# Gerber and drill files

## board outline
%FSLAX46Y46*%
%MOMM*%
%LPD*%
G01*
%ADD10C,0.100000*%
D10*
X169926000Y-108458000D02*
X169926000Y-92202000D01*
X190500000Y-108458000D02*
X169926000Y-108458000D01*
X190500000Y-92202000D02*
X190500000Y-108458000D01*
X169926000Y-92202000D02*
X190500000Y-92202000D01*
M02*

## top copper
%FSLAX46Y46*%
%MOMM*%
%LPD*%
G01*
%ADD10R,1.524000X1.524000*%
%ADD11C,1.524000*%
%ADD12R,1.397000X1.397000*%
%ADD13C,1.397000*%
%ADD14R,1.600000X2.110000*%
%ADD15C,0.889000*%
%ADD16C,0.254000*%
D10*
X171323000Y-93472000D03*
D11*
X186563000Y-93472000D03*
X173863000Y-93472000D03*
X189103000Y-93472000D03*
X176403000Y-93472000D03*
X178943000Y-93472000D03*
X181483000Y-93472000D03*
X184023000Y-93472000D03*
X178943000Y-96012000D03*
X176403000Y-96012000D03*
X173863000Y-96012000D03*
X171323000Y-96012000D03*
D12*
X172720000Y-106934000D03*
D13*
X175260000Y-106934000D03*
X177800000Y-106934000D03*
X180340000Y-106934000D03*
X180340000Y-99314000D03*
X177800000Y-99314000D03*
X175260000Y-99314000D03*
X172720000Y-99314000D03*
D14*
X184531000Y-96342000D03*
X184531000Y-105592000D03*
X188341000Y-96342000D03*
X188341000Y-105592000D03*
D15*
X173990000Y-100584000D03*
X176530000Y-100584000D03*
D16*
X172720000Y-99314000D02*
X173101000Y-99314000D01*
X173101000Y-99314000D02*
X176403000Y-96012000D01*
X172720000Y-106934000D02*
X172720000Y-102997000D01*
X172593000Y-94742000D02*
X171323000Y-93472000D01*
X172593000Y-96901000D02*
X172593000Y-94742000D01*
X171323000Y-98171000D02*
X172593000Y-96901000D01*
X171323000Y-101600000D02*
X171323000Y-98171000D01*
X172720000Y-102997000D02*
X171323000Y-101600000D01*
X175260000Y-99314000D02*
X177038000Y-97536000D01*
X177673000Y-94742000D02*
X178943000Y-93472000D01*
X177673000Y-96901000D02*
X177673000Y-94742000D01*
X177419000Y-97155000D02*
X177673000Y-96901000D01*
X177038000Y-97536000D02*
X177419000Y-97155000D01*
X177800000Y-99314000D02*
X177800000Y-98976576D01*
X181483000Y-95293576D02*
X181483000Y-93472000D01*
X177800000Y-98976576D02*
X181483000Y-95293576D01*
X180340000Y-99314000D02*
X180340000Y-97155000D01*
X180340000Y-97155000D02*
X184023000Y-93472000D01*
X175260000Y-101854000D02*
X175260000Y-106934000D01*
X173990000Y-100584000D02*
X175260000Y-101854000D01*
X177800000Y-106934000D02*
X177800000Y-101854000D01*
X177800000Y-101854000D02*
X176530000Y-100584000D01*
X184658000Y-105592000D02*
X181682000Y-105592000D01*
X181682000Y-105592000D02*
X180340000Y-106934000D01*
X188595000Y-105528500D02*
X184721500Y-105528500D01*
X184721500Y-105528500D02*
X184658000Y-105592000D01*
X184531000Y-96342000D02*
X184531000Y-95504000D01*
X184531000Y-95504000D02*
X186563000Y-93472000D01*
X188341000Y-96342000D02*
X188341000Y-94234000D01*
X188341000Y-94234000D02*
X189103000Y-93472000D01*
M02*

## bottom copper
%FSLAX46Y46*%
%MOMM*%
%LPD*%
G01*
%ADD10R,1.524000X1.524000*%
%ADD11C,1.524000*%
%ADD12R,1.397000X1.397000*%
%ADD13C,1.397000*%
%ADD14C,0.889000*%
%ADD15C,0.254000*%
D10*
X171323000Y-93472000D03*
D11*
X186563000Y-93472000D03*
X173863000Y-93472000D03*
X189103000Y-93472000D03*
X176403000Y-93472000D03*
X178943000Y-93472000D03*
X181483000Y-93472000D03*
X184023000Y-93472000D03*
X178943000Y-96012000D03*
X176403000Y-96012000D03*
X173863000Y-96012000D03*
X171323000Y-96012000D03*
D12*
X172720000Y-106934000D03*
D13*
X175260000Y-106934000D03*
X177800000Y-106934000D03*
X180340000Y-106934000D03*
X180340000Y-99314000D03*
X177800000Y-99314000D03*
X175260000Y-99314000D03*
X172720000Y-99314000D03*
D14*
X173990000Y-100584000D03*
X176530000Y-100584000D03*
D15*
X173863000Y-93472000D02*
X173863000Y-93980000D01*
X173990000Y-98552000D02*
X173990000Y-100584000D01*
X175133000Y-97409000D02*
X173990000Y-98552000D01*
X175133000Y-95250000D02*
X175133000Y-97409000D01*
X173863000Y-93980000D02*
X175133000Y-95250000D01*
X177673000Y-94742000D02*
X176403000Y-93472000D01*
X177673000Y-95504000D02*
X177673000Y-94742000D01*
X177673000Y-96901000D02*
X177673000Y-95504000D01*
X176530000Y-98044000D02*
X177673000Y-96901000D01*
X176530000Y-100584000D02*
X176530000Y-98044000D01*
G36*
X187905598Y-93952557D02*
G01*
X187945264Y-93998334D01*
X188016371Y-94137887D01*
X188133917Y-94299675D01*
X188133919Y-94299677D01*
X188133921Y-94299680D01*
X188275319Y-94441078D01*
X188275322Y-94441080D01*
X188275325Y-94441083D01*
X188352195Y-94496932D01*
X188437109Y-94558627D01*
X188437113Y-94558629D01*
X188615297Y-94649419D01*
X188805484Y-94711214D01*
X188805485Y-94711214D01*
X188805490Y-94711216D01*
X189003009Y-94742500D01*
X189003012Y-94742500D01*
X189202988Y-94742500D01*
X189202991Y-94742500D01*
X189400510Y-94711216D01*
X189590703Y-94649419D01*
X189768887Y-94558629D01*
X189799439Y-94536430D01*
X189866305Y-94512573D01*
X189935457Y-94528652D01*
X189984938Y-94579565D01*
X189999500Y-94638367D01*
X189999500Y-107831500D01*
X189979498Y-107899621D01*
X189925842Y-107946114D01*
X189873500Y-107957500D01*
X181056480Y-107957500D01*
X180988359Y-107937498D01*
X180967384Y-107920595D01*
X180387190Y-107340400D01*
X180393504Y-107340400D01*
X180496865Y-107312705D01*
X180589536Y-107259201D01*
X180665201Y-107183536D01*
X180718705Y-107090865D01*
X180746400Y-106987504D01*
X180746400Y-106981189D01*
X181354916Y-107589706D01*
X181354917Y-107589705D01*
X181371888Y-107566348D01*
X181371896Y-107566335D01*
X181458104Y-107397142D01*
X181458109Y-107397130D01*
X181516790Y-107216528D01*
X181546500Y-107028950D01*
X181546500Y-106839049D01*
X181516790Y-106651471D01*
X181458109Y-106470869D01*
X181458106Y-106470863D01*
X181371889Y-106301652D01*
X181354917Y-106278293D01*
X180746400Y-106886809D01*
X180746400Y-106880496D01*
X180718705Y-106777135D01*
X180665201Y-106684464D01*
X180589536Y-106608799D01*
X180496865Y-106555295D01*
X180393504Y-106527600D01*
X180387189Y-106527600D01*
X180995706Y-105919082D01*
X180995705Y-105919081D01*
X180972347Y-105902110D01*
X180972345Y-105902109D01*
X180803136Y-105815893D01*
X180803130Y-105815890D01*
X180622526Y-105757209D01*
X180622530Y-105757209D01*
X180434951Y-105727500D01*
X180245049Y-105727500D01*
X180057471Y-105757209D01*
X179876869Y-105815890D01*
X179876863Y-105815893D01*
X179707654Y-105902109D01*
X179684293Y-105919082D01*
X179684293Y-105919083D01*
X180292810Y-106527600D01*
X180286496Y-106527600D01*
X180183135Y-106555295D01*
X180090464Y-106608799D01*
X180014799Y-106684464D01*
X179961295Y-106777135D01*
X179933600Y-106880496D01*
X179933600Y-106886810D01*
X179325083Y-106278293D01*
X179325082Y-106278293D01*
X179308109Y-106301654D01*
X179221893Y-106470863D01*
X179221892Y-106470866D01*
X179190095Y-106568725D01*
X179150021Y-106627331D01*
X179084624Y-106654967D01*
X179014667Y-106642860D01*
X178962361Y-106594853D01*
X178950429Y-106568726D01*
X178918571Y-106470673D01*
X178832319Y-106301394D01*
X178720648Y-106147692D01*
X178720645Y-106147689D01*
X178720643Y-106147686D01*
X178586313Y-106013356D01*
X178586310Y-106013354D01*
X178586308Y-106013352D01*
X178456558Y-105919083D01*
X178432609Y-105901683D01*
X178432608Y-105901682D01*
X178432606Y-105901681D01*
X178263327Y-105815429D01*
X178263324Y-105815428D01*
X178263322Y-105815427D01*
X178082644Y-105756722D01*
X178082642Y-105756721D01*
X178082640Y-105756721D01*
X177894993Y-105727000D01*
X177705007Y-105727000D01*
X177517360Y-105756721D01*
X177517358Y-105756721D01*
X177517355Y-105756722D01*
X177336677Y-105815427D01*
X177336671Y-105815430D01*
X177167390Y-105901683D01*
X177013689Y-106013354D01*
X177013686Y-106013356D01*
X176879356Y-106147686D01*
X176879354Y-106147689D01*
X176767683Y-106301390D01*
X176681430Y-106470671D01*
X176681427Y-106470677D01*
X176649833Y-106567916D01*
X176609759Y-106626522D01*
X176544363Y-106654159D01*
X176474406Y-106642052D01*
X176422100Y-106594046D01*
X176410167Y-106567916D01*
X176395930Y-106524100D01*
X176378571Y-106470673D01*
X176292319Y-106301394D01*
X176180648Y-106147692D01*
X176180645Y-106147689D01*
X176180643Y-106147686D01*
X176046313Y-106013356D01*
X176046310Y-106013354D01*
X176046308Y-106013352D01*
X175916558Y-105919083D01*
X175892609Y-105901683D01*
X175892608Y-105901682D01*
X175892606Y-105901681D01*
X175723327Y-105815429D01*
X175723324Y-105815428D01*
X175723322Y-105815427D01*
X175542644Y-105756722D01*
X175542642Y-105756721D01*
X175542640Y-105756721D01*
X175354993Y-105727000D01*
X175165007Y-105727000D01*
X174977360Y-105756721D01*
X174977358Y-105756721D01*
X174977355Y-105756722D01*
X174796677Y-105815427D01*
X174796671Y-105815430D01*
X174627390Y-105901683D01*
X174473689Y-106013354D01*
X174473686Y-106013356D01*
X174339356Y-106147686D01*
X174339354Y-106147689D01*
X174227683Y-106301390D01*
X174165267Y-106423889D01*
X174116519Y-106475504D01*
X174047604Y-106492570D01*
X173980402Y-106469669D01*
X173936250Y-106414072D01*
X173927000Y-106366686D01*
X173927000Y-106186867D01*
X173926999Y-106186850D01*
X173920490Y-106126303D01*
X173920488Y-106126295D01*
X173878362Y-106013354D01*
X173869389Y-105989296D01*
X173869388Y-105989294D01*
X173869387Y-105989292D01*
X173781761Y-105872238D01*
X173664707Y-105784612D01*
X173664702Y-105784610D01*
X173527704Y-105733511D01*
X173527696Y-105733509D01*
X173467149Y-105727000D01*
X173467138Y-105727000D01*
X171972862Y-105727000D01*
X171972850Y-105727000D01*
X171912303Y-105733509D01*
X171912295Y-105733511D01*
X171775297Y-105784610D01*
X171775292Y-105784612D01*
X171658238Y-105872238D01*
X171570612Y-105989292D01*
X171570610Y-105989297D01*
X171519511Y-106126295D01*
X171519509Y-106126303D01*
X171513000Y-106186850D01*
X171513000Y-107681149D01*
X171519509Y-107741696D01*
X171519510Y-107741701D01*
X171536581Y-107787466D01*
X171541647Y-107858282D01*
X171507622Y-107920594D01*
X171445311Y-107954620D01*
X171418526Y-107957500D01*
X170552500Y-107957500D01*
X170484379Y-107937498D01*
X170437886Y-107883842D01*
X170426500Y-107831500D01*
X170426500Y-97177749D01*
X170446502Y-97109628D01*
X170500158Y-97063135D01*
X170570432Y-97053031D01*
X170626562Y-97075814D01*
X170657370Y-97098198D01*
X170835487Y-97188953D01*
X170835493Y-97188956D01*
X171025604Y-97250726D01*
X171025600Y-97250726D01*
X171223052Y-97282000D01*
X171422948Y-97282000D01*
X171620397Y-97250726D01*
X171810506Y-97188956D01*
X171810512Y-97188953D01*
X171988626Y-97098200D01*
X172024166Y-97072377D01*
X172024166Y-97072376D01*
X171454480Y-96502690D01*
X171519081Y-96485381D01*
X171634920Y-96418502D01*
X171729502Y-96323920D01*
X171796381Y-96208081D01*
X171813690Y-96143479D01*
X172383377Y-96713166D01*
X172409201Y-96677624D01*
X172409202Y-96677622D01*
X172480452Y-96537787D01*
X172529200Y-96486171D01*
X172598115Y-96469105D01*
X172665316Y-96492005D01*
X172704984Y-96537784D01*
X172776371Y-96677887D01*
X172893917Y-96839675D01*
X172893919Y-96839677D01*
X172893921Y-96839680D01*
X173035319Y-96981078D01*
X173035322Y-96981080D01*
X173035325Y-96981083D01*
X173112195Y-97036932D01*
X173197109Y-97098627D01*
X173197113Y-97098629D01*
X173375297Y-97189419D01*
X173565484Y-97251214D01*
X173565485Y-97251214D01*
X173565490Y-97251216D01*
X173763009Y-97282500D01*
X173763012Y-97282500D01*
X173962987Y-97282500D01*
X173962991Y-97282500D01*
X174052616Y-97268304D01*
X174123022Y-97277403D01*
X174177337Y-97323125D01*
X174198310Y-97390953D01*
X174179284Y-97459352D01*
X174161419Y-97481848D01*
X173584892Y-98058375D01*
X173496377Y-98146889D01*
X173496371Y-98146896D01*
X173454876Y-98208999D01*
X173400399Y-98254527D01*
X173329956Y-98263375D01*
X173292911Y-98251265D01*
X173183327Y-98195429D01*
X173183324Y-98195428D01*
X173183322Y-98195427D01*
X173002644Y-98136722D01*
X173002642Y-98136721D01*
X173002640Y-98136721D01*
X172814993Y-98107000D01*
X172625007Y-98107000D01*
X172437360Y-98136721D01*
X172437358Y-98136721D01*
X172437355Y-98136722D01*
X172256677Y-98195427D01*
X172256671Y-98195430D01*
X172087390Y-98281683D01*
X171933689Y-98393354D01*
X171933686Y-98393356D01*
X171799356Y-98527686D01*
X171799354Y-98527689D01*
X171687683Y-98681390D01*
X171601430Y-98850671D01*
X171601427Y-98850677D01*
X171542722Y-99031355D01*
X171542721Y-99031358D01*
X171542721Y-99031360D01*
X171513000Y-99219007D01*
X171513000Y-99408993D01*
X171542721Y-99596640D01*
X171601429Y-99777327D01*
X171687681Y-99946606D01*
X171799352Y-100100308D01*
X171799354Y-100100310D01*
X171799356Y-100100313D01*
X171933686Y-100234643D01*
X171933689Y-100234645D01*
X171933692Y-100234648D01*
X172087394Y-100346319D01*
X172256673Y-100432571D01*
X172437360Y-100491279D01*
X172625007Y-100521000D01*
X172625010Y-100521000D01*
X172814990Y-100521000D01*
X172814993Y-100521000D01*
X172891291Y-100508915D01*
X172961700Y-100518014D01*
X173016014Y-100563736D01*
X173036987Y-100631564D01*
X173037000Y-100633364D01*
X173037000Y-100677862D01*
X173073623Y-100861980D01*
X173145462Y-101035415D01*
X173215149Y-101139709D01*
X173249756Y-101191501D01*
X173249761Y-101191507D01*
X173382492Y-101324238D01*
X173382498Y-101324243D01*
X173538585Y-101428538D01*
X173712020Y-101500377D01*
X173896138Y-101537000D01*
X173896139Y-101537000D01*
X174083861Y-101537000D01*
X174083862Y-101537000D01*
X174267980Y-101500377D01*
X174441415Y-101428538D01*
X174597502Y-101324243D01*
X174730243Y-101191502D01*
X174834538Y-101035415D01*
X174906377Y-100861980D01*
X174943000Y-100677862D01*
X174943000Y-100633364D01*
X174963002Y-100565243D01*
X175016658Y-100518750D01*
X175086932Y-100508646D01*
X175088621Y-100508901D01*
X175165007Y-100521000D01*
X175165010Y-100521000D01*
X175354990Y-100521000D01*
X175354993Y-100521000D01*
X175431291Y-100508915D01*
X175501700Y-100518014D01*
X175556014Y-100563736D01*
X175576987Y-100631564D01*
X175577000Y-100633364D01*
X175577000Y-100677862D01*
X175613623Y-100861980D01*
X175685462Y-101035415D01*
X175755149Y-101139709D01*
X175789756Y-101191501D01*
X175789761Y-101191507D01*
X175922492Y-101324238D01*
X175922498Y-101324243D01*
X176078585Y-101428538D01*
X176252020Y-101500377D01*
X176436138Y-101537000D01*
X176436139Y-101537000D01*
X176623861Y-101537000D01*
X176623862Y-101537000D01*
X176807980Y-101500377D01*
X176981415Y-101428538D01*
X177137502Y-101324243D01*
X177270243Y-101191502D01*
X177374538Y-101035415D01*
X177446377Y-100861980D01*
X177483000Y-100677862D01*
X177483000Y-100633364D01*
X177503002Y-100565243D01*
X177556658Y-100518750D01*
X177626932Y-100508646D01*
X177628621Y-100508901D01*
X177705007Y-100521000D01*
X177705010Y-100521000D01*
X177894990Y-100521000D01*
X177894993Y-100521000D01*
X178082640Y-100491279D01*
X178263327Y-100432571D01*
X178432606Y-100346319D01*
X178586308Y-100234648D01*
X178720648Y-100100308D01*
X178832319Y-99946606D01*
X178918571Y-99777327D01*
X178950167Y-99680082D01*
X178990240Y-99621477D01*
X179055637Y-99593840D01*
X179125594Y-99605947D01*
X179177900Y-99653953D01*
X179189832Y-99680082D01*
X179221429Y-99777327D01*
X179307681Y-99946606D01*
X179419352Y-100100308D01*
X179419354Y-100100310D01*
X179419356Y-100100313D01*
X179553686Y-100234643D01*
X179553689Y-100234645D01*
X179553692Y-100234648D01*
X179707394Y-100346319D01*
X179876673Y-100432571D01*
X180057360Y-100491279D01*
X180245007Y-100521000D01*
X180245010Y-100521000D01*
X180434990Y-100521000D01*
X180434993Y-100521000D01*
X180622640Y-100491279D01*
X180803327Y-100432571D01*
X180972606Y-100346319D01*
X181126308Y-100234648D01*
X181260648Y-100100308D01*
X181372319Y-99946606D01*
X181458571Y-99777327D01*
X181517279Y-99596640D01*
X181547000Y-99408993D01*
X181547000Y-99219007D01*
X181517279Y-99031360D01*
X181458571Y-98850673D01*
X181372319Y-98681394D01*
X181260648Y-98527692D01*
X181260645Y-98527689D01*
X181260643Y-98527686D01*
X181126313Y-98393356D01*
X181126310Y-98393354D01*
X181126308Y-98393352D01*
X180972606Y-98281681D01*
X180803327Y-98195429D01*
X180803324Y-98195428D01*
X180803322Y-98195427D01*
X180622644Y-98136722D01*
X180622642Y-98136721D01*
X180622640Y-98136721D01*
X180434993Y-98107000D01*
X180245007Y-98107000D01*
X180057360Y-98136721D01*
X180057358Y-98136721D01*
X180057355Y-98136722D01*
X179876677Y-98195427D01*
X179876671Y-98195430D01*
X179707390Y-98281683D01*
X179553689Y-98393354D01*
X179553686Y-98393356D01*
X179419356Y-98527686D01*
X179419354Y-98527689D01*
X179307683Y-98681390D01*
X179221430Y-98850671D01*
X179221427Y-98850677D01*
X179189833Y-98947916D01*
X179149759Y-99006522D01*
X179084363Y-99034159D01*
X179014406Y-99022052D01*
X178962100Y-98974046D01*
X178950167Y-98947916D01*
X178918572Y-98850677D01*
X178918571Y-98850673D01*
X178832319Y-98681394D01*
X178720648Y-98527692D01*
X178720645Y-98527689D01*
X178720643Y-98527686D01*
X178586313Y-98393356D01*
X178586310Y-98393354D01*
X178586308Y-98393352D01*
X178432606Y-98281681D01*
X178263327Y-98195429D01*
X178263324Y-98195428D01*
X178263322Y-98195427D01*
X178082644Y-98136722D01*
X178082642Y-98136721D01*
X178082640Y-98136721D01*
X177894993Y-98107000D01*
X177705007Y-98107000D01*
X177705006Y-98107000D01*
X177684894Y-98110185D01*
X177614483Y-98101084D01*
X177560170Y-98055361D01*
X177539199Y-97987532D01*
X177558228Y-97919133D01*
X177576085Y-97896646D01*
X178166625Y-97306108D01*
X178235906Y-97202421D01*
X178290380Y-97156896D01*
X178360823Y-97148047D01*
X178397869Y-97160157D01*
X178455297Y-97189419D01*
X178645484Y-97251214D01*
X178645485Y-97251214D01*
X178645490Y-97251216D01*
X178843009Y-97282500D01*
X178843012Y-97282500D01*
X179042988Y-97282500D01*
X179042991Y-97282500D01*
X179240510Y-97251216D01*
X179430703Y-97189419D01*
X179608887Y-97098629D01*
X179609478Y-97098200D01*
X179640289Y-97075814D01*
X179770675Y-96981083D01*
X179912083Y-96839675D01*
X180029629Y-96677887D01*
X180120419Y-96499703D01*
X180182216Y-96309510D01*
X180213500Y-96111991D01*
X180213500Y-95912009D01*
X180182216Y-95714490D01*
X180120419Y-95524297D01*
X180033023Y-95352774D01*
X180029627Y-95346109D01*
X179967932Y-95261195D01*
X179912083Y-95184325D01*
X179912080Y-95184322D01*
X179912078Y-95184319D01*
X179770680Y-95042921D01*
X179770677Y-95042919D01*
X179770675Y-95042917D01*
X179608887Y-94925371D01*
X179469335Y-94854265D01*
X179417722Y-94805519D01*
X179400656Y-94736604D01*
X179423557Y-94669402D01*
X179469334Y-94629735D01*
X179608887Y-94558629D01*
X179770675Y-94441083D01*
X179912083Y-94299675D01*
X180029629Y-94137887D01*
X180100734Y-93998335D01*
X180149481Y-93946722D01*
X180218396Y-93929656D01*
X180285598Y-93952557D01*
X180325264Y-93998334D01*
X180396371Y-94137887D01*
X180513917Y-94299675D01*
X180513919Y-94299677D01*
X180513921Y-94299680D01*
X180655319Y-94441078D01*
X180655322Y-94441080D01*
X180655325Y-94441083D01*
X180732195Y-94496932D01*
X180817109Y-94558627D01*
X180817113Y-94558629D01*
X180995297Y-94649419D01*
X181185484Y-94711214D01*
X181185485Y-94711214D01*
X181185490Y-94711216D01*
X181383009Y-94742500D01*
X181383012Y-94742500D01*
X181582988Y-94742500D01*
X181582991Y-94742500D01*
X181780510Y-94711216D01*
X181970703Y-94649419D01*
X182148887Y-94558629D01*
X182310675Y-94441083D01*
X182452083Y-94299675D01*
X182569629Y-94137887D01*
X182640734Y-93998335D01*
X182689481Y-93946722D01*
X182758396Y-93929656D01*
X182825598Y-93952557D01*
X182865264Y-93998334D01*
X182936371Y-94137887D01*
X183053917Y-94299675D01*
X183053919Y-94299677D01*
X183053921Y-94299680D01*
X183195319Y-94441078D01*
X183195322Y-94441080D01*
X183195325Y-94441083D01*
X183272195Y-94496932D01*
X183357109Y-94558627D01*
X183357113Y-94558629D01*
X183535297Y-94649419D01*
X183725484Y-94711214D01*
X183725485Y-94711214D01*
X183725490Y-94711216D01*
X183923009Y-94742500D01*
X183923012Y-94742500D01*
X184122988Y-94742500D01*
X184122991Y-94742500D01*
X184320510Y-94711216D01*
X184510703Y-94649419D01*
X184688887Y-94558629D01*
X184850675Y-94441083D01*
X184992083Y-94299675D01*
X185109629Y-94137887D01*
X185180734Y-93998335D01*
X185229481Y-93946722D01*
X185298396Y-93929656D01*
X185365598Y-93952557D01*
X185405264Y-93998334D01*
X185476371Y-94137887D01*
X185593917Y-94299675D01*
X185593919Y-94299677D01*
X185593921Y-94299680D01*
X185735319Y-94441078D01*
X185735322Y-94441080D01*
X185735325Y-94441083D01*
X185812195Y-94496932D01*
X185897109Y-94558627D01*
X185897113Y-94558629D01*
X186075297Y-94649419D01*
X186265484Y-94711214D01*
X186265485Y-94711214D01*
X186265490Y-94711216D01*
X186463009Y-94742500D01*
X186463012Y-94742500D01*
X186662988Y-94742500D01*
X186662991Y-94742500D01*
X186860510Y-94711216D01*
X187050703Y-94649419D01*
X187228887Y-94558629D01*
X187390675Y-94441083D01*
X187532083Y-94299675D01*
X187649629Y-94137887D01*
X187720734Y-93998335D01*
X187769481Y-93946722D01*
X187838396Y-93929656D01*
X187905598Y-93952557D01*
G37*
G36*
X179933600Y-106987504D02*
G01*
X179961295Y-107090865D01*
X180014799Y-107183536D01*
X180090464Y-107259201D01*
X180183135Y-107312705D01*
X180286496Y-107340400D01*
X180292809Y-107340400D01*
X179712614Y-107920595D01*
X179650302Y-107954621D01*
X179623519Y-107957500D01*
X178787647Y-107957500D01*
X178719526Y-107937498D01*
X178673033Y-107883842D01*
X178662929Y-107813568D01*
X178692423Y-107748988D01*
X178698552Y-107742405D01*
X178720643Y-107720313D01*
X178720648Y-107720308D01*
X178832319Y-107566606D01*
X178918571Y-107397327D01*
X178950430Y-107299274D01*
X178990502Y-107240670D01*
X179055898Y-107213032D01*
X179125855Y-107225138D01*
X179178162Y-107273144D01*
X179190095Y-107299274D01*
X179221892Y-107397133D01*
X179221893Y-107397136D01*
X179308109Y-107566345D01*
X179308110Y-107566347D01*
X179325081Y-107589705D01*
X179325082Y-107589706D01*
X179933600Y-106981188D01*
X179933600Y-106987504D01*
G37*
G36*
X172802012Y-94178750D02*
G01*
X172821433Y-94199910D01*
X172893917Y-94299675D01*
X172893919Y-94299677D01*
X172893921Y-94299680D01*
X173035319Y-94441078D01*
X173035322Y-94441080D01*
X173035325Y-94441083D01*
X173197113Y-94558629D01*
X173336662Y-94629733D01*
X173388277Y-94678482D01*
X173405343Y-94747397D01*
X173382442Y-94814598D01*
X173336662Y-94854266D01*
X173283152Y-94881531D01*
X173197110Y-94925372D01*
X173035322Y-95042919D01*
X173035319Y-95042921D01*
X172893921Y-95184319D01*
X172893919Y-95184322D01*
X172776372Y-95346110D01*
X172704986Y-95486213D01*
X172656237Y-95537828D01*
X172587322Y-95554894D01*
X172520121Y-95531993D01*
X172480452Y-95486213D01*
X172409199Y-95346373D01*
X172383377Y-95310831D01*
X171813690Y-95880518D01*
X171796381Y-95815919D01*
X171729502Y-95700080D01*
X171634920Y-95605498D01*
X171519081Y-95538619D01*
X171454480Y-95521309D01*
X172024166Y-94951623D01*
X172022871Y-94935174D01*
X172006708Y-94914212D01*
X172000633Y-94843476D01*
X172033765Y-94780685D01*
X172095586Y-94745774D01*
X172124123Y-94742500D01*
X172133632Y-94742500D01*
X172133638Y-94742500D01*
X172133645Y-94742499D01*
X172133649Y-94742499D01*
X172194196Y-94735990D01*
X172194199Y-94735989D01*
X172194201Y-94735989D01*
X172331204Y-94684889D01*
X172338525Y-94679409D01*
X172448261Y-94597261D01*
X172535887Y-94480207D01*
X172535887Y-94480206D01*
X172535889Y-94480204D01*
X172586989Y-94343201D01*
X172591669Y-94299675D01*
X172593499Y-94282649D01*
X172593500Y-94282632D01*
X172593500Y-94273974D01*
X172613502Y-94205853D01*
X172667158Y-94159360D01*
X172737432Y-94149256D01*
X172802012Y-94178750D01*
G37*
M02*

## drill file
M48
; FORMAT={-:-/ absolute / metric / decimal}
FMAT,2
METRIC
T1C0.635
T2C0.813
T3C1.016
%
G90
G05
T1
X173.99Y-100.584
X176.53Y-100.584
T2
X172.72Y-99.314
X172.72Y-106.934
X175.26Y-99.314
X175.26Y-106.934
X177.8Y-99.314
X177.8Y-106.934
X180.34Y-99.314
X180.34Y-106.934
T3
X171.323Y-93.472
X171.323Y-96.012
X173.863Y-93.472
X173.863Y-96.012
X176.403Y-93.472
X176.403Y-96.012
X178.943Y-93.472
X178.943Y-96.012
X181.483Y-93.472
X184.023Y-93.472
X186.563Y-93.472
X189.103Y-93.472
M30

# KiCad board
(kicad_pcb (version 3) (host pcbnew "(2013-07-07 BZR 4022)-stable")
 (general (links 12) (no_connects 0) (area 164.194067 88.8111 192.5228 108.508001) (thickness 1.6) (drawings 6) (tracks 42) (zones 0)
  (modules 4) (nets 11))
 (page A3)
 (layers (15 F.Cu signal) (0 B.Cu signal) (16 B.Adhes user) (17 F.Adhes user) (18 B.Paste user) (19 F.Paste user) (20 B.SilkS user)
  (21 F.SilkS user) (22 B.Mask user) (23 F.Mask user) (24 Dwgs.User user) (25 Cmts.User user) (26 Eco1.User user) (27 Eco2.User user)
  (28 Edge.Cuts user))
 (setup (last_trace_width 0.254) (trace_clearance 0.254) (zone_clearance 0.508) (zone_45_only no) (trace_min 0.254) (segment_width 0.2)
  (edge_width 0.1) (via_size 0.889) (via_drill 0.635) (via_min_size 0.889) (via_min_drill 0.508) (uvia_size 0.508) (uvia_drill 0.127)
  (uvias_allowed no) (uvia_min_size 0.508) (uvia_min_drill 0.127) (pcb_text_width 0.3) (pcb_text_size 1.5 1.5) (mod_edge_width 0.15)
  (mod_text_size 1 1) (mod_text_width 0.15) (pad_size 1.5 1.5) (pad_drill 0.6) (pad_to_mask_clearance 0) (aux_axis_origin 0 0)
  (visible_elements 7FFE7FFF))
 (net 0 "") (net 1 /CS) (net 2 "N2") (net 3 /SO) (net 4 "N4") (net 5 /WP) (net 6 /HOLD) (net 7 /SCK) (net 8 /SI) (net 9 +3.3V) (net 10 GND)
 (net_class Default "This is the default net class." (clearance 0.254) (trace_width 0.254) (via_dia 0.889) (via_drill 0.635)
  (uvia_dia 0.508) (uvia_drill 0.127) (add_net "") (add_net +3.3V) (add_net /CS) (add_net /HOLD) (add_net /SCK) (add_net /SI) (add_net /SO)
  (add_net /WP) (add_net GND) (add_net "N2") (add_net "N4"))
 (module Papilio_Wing (layer F.Cu) (at 171.323 93.472)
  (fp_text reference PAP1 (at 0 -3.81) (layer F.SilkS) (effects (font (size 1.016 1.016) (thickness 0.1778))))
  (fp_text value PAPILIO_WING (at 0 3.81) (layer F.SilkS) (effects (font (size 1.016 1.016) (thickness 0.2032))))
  (pad 1 thru_hole rect (at 0 0) (size 1.524 1.524) (drill 1.016) (layers *.Cu *.Mask F.SilkS) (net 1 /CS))
  (pad 7 thru_hole circle (at 15.24 0) (size 1.524 1.524) (drill 1.016) (layers *.Cu *.Mask F.SilkS) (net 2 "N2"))
  (pad 2 thru_hole circle (at 2.54 0) (size 1.524 1.524) (drill 1.016) (layers *.Cu *.Mask F.SilkS) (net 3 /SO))
  (pad 8 thru_hole circle (at 17.78 0) (size 1.524 1.524) (drill 1.016) (layers *.Cu *.Mask F.SilkS) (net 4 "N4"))
  (pad 3 thru_hole circle (at 5.08 0) (size 1.524 1.524) (drill 1.016) (layers *.Cu *.Mask F.SilkS) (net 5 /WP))
  (pad 4 thru_hole circle (at 7.62 0) (size 1.524 1.524) (drill 1.016) (layers *.Cu *.Mask F.SilkS) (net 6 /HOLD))
  (pad 5 thru_hole circle (at 10.16 0) (size 1.524 1.524) (drill 1.016) (layers *.Cu *.Mask F.SilkS) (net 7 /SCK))
  (pad 6 thru_hole circle (at 12.7 0) (size 1.524 1.524) (drill 1.016) (layers *.Cu *.Mask F.SilkS) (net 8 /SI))
  (pad 9 thru_hole circle (at 7.62 2.54) (size 1.524 1.524) (drill 1.016) (layers *.Cu *.Mask F.SilkS))
  (pad 10 thru_hole circle (at 5.08 2.54) (size 1.524 1.524) (drill 1.016) (layers *.Cu *.Mask F.SilkS) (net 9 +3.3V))
  (pad 11 thru_hole circle (at 2.54 2.54) (size 1.524 1.524) (drill 1.016) (layers *.Cu *.Mask F.SilkS))
  (pad 12 thru_hole circle (at 0 2.54) (size 1.524 1.524) (drill 1.016) (layers *.Cu *.Mask F.SilkS) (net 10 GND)))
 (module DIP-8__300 (layer F.Cu) (at 176.53 103.124)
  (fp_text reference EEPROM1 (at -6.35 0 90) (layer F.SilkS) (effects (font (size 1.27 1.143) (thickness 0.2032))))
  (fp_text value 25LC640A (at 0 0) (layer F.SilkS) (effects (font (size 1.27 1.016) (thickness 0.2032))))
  (pad 1 thru_hole rect (at -3.81 3.81) (size 1.397 1.397) (drill 0.8128) (layers *.Cu *.Mask F.SilkS) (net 1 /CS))
  (pad 2 thru_hole circle (at -1.27 3.81) (size 1.397 1.397) (drill 0.8128) (layers *.Cu *.Mask F.SilkS) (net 3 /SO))
  (pad 3 thru_hole circle (at 1.27 3.81) (size 1.397 1.397) (drill 0.8128) (layers *.Cu *.Mask F.SilkS) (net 5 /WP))
  (pad 4 thru_hole circle (at 3.81 3.81) (size 1.397 1.397) (drill 0.8128) (layers *.Cu *.Mask F.SilkS) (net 10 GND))
  (pad 5 thru_hole circle (at 3.81 -3.81) (size 1.397 1.397) (drill 0.8128) (layers *.Cu *.Mask F.SilkS) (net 8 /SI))
  (pad 6 thru_hole circle (at 1.27 -3.81) (size 1.397 1.397) (drill 0.8128) (layers *.Cu *.Mask F.SilkS) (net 7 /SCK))
  (pad 7 thru_hole circle (at -1.27 -3.81) (size 1.397 1.397) (drill 0.8128) (layers *.Cu *.Mask F.SilkS) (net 6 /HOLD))
  (pad 8 thru_hole circle (at -3.81 -3.81) (size 1.397 1.397) (drill 0.8128) (layers *.Cu *.Mask F.SilkS) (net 9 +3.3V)))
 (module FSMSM (layer F.Cu) (at 184.531 101.092 270)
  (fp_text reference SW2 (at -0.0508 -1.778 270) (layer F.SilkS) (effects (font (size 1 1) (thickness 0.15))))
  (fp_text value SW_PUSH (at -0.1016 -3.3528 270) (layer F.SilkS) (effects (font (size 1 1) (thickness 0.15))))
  (pad 1 smd rect (at -4.75 0 270) (size 2.11 1.6) (layers F.Cu F.Paste F.Mask) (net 2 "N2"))
  (pad 2 smd rect (at 4.5 0 270) (size 2.11 1.6) (layers F.Cu F.Paste F.Mask) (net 10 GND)))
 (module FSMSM (layer F.Cu) (at 188.341 101.092 270)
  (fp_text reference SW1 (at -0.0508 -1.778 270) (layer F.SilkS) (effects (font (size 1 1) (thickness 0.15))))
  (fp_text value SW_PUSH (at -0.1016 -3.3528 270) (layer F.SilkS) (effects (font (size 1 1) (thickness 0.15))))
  (pad 1 smd rect (at -4.75 0 270) (size 2.11 1.6) (layers F.Cu F.Paste F.Mask) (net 4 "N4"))
  (pad 2 smd rect (at 4.5 0 270) (size 2.11 1.6) (layers F.Cu F.Paste F.Mask) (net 10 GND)))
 (gr_line (start 169.926 108.458) (end 169.926 92.202) (angle 90) (layer Edge.Cuts) (width 0.1))
 (gr_line (start 190.5 108.458) (end 169.926 108.458) (angle 90) (layer Edge.Cuts) (width 0.1))
 (gr_line (start 190.5 92.202) (end 190.5 108.458) (angle 90) (layer Edge.Cuts) (width 0.1))
 (gr_line (start 169.926 92.202) (end 190.5 92.202) (angle 90) (layer Edge.Cuts) (width 0.1))
 (segment (start 172.72 99.314) (end 173.101 99.314) (width 0.254) (layer F.Cu) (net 9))
 (segment (start 173.101 99.314) (end 176.403 96.012) (width 0.254) (layer F.Cu) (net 9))
 (segment (start 172.72 106.934) (end 172.72 102.997) (width 0.254) (layer F.Cu) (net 1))
 (segment (start 172.593 94.742) (end 171.323 93.472) (width 0.254) (layer F.Cu) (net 1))
 (segment (start 172.593 96.901) (end 172.593 94.742) (width 0.254) (layer F.Cu) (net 1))
 (segment (start 171.323 98.171) (end 172.593 96.901) (width 0.254) (layer F.Cu) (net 1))
 (segment (start 171.323 101.6) (end 171.323 98.171) (width 0.254) (layer F.Cu) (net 1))
 (segment (start 172.72 102.997) (end 171.323 101.6) (width 0.254) (layer F.Cu) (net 1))
 (segment (start 175.26 99.314) (end 177.038 97.536) (width 0.254) (layer F.Cu) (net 6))
 (segment (start 177.673 94.742) (end 178.943 93.472) (width 0.254) (layer F.Cu) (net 6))
 (segment (start 177.673 96.901) (end 177.673 94.742) (width 0.254) (layer F.Cu) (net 6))
 (segment (start 177.419 97.155) (end 177.673 96.901) (width 0.254) (layer F.Cu) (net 6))
 (segment (start 177.038 97.536) (end 177.419 97.155) (width 0.254) (layer F.Cu) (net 6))
 (segment (start 177.8 99.314) (end 177.8 98.976576) (width 0.254) (layer F.Cu) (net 7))
 (segment (start 181.483 95.293576) (end 181.483 93.472) (width 0.254) (layer F.Cu) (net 7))
 (segment (start 177.8 98.976576) (end 181.483 95.293576) (width 0.254) (layer F.Cu) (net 7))
 (segment (start 180.34 99.314) (end 180.34 97.155) (width 0.254) (layer F.Cu) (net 8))
 (segment (start 180.34 97.155) (end 184.023 93.472) (width 0.254) (layer F.Cu) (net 8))
 (segment (start 173.863 93.472) (end 173.863 93.98) (width 0.254) (layer B.Cu) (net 3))
 (segment (start 175.26 101.854) (end 175.26 106.934) (width 0.254) (layer F.Cu) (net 3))
 (segment (start 173.99 100.584) (end 175.26 101.854) (width 0.254) (layer F.Cu) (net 3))
 (via (at 173.99 100.584) (size 0.889) (layers F.Cu B.Cu) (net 3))
 (segment (start 173.99 98.552) (end 173.99 100.584) (width 0.254) (layer B.Cu) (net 3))
 (segment (start 175.133 97.409) (end 173.99 98.552) (width 0.254) (layer B.Cu) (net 3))
 (segment (start 175.133 95.25) (end 175.133 97.409) (width 0.254) (layer B.Cu) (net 3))
 (segment (start 173.863 93.98) (end 175.133 95.25) (width 0.254) (layer B.Cu) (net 3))
 (segment (start 177.8 106.934) (end 177.8 101.854) (width 0.254) (layer F.Cu) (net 5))
 (segment (start 177.673 94.742) (end 176.403 93.472) (width 0.254) (layer B.Cu) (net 5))
 (segment (start 177.673 95.504) (end 177.673 94.742) (width 0.254) (layer B.Cu) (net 5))
 (segment (start 177.673 96.901) (end 177.673 95.504) (width 0.254) (layer B.Cu) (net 5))
 (segment (start 176.53 98.044) (end 177.673 96.901) (width 0.254) (layer B.Cu) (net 5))
 (segment (start 176.53 100.584) (end 176.53 98.044) (width 0.254) (layer B.Cu) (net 5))
 (via (at 176.53 100.584) (size 0.889) (layers F.Cu B.Cu) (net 5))
 (segment (start 177.8 101.854) (end 176.53 100.584) (width 0.254) (layer F.Cu) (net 5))
 (segment (start 184.658 105.592) (end 181.682 105.592) (width 0.254) (layer F.Cu) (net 10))
 (segment (start 181.682 105.592) (end 180.34 106.934) (width 0.254) (layer F.Cu) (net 10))
 (segment (start 188.595 105.5285) (end 184.7215 105.5285) (width 0.254) (layer F.Cu) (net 10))
 (segment (start 184.7215 105.5285) (end 184.658 105.592) (width 0.254) (layer F.Cu) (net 10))
 (segment (start 184.531 96.342) (end 184.531 95.504) (width 0.254) (layer F.Cu) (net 2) (status C00000))
 (segment (start 184.531 95.504) (end 186.563 93.472) (width 0.254) (layer F.Cu) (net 2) (status C00000))
 (segment (start 188.341 96.342) (end 188.341 94.234) (width 0.254) (layer F.Cu) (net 4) (status 400000))
 (segment (start 188.341 94.234) (end 189.103 93.472) (width 0.254) (layer F.Cu) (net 4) (status 800000))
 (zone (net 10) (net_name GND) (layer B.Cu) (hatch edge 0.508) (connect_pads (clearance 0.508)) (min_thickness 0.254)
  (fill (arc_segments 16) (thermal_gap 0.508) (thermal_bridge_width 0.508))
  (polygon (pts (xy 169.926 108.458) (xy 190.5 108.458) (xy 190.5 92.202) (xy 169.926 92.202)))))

